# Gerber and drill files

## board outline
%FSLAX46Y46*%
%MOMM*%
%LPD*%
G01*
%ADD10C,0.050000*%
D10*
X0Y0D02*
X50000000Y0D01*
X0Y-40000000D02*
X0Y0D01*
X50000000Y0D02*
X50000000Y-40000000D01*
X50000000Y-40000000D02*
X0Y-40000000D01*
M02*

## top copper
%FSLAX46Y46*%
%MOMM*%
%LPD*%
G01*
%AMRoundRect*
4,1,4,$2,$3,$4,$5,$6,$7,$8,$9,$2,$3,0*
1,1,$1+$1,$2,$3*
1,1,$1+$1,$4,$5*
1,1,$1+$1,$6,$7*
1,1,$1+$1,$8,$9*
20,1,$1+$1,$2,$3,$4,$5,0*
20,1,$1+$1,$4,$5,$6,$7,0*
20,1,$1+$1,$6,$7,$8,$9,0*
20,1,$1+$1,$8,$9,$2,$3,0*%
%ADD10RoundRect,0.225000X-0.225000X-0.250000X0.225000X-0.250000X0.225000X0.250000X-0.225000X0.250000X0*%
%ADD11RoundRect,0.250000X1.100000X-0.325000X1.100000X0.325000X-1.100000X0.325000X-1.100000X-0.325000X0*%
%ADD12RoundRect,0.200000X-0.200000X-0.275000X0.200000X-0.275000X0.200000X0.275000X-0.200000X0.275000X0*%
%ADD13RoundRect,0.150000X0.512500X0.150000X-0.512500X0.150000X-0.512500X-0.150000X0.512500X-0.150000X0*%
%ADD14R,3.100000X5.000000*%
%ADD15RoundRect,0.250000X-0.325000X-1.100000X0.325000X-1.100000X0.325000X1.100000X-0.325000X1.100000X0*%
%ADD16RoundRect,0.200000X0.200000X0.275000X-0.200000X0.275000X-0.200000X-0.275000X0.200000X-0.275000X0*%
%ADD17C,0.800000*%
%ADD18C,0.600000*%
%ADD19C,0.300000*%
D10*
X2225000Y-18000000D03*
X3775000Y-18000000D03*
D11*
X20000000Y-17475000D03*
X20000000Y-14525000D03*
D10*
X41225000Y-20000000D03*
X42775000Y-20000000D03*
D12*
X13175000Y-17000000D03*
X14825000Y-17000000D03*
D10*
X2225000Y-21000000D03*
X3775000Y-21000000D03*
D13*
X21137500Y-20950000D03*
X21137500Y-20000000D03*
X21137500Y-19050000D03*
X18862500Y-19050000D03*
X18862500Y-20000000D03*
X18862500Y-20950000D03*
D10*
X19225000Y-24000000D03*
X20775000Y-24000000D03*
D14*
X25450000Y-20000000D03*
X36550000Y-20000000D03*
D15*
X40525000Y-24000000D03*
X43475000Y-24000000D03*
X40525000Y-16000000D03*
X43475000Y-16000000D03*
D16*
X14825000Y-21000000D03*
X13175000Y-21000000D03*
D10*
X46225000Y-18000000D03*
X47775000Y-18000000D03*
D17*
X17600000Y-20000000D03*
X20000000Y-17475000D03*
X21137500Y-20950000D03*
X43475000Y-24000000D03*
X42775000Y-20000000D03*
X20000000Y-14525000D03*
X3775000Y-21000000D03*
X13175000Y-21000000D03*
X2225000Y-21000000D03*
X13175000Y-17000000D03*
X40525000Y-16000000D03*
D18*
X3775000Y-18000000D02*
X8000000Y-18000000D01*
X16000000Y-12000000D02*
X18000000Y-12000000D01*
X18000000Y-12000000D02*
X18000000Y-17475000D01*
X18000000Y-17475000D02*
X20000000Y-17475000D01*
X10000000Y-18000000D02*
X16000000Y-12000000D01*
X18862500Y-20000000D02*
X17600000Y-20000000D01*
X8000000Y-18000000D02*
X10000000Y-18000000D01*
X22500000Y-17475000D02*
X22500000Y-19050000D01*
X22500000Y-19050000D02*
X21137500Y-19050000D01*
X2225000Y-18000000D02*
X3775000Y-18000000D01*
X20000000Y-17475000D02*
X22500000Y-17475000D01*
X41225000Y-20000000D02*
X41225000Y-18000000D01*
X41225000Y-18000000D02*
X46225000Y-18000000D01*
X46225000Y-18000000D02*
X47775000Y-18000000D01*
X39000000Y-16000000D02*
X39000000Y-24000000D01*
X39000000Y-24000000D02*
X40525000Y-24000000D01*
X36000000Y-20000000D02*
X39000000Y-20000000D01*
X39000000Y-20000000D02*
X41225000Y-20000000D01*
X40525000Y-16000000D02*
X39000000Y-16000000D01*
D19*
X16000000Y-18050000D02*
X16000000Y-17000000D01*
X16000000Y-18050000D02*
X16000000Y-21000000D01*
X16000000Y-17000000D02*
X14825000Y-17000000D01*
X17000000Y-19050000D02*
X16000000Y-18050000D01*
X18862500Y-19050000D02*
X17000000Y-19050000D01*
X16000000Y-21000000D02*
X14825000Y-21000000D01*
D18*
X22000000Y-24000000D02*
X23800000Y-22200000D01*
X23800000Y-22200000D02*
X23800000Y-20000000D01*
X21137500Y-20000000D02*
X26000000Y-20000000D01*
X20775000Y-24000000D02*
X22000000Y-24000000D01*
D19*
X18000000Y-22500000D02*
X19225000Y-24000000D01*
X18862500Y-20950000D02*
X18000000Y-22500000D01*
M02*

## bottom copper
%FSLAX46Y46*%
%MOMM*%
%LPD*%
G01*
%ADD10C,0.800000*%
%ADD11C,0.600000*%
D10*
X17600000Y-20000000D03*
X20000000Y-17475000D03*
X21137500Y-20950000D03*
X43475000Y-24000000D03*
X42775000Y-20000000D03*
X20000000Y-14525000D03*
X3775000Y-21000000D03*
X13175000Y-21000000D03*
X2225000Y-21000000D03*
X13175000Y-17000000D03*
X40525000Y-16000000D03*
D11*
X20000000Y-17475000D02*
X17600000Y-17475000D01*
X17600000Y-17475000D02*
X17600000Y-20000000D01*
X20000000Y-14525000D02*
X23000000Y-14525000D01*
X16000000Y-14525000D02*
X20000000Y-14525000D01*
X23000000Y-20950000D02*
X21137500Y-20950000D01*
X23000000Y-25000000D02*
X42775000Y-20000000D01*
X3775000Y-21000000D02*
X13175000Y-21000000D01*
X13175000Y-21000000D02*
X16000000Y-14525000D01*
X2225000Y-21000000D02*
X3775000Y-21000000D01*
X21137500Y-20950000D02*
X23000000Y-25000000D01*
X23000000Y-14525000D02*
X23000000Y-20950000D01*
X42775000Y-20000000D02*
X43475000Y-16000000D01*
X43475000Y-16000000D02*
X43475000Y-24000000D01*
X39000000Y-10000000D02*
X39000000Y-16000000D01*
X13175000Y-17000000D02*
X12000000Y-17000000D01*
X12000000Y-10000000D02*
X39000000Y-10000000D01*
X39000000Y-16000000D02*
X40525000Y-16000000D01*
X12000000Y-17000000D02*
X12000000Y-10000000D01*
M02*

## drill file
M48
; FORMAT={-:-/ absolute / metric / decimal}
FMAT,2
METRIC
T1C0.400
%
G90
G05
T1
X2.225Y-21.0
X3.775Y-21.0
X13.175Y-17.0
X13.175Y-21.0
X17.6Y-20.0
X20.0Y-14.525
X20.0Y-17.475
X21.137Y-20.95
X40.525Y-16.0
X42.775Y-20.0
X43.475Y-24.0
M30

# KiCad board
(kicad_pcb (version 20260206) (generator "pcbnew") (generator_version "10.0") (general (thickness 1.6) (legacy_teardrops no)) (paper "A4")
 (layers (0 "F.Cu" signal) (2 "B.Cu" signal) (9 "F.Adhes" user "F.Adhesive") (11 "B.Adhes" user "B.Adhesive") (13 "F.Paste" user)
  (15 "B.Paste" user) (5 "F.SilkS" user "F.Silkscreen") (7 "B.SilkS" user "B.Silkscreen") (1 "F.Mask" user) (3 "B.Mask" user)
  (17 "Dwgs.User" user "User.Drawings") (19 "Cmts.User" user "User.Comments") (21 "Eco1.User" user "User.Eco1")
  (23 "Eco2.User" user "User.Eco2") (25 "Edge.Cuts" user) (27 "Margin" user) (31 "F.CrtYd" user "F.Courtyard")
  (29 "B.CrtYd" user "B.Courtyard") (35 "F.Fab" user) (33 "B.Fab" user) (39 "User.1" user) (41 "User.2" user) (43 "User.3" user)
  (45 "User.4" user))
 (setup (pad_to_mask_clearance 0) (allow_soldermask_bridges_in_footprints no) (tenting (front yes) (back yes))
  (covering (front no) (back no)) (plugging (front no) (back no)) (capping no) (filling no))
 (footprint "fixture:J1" (layer "F.Cu") (at 3 18)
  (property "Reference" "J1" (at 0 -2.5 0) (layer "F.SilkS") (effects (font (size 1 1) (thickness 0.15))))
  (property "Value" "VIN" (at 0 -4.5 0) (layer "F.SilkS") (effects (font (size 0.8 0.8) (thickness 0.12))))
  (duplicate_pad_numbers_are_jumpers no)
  (pad "1" smd roundrect (at -0.775 0) (size 0.9 0.95) (layers "F.Cu" "F.Mask" "F.Paste") (roundrect_rratio 0.25) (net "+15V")
   (thermal_bridge_angle 45))
  (pad "2" smd roundrect (at 0.775 0) (size 0.9 0.95) (layers "F.Cu" "F.Mask" "F.Paste") (roundrect_rratio 0.25) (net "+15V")
   (thermal_bridge_angle 45)))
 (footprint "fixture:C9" (layer "F.Cu") (at 20 16 90)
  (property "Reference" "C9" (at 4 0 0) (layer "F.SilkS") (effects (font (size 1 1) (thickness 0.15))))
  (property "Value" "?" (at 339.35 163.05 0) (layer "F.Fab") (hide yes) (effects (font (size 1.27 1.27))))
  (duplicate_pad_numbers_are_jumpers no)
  (pad "1" smd roundrect (at -1.475 0 90) (size 1.15 2.7) (layers "F.Cu" "F.Mask" "F.Paste") (roundrect_rratio 0.217391) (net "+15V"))
  (pad "2" smd roundrect (at 1.475 0 90) (size 1.15 2.7) (layers "F.Cu" "F.Mask" "F.Paste") (roundrect_rratio 0.217391) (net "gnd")))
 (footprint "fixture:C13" (layer "F.Cu") (at 42 20)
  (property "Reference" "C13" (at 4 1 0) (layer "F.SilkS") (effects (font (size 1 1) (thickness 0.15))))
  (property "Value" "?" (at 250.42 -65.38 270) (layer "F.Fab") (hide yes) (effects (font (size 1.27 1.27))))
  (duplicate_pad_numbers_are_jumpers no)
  (pad "1" smd roundrect (at -0.775 0) (size 0.9 0.95) (layers "F.Cu" "F.Mask" "F.Paste") (roundrect_rratio 0.25) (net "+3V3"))
  (pad "2" smd roundrect (at 0.775 0) (size 0.9 0.95) (layers "F.Cu" "F.Mask" "F.Paste") (roundrect_rratio 0.25) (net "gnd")))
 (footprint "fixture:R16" (layer "F.Cu") (at 14 17)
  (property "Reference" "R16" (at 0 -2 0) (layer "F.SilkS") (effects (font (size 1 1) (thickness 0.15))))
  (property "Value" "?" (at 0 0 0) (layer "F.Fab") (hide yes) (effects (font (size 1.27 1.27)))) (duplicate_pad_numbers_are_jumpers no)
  (pad "1" smd roundrect (at -0.825 0) (size 0.8 0.95) (layers "F.Cu" "F.Mask" "F.Paste") (roundrect_rratio 0.25) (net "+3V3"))
  (pad "2" smd roundrect (at 0.825 0) (size 0.8 0.95) (layers "F.Cu" "F.Mask" "F.Paste") (roundrect_rratio 0.25) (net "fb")))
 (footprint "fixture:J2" (layer "F.Cu") (at 3 21)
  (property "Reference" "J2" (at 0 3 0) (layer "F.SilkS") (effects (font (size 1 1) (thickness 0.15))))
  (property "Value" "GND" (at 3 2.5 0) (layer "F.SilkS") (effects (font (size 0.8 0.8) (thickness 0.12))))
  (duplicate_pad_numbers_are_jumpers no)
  (pad "1" smd roundrect (at -0.775 0) (size 0.9 0.95) (layers "F.Cu" "F.Mask" "F.Paste") (roundrect_rratio 0.25) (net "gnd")
   (thermal_bridge_angle 45))
  (pad "2" smd roundrect (at 0.775 0) (size 0.9 0.95) (layers "F.Cu" "F.Mask" "F.Paste") (roundrect_rratio 0.25) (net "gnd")
   (thermal_bridge_angle 45)))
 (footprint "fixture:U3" (layer "F.Cu") (at 20 20 180)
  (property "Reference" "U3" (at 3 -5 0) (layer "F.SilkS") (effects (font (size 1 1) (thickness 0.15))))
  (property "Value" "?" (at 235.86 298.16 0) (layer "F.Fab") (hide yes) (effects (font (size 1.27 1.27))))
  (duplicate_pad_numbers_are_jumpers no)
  (pad "1" smd roundrect (at -1.1375 -0.95 180) (size 1.325 0.6) (layers "F.Cu" "F.Mask" "F.Paste") (roundrect_rratio 0.25) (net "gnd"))
  (pad "2" smd roundrect (at -1.1375 0 180) (size 1.325 0.6) (layers "F.Cu" "F.Mask" "F.Paste") (roundrect_rratio 0.25) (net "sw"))
  (pad "3" smd roundrect (at -1.1375 0.95 180) (size 1.325 0.6) (layers "F.Cu" "F.Mask" "F.Paste") (roundrect_rratio 0.25) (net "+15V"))
  (pad "4" smd roundrect (at 1.1375 0.95 180) (size 1.325 0.6) (layers "F.Cu" "F.Mask" "F.Paste") (roundrect_rratio 0.25) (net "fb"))
  (pad "5" smd roundrect (at 1.1375 0 180) (size 1.325 0.6) (layers "F.Cu" "F.Mask" "F.Paste") (roundrect_rratio 0.25) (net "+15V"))
  (pad "6" smd roundrect (at 1.1375 -0.95 180) (size 1.325 0.6) (layers "F.Cu" "F.Mask" "F.Paste") (roundrect_rratio 0.25) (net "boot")))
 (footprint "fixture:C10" (layer "F.Cu") (at 20 24)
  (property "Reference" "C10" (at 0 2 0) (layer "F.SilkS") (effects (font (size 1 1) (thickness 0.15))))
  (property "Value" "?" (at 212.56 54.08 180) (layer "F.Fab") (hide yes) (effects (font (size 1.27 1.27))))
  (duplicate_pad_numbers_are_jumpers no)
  (pad "1" smd roundrect (at -0.775 0) (size 0.9 0.95) (layers "F.Cu" "F.Mask" "F.Paste") (roundrect_rratio 0.25) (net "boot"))
  (pad "2" smd roundrect (at 0.775 0) (size 0.9 0.95) (layers "F.Cu" "F.Mask" "F.Paste") (roundrect_rratio 0.25) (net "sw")))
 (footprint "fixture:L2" (layer "F.Cu") (at 31 20)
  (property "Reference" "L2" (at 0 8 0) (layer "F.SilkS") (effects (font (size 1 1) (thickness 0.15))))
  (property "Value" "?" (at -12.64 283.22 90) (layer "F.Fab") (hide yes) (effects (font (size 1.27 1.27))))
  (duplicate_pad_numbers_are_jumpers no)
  (pad "1" smd rect (at -5.55 0) (size 3.1 5) (layers "F.Cu" "F.Mask" "F.Paste") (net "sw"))
  (pad "2" smd rect (at 5.55 0) (size 3.1 5) (layers "F.Cu" "F.Mask" "F.Paste") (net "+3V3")))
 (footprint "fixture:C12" (layer "F.Cu") (at 42 24)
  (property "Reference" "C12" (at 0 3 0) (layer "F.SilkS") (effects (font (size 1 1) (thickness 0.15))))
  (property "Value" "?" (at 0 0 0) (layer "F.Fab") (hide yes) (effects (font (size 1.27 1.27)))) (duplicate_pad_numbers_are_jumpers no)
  (pad "1" smd roundrect (at -1.475 0) (size 1.15 2.7) (layers "F.Cu" "F.Mask" "F.Paste") (roundrect_rratio 0.217391) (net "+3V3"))
  (pad "2" smd roundrect (at 1.475 0) (size 1.15 2.7) (layers "F.Cu" "F.Mask" "F.Paste") (roundrect_rratio 0.217391) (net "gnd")))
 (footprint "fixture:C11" (layer "F.Cu") (at 42 16)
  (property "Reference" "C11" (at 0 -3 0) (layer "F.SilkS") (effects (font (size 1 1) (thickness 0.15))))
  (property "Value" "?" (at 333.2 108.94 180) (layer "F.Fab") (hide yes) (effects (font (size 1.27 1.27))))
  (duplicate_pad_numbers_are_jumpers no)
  (pad "1" smd roundrect (at -1.475 0) (size 1.15 2.7) (layers "F.Cu" "F.Mask" "F.Paste") (roundrect_rratio 0.217391) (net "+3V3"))
  (pad "2" smd roundrect (at 1.475 0) (size 1.15 2.7) (layers "F.Cu" "F.Mask" "F.Paste") (roundrect_rratio 0.217391) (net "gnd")))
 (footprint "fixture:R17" (layer "F.Cu") (at 14 21 180)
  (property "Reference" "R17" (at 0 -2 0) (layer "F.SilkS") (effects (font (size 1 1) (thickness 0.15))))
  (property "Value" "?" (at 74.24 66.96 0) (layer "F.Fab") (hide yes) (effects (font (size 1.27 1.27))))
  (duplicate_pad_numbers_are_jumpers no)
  (pad "1" smd roundrect (at -0.825 0 180) (size 0.8 0.95) (layers "F.Cu" "F.Mask" "F.Paste") (roundrect_rratio 0.25) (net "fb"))
  (pad "2" smd roundrect (at 0.825 0 180) (size 0.8 0.95) (layers "F.Cu" "F.Mask" "F.Paste") (roundrect_rratio 0.25) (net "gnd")))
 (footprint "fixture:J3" (layer "F.Cu") (at 47 18)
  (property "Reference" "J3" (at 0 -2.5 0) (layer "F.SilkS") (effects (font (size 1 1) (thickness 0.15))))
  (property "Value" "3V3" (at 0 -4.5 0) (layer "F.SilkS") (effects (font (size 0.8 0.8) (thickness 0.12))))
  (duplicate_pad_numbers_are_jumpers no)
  (pad "1" smd roundrect (at -0.775 0) (size 0.9 0.95) (layers "F.Cu" "F.Mask" "F.Paste") (roundrect_rratio 0.25) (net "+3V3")
   (thermal_bridge_angle 45))
  (pad "2" smd roundrect (at 0.775 0) (size 0.9 0.95) (layers "F.Cu" "F.Mask" "F.Paste") (roundrect_rratio 0.25) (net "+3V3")
   (thermal_bridge_angle 45)))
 (gr_line (start 0 0) (end 50 0) (stroke (width 0.05) (type default)) (layer "Edge.Cuts"))
 (gr_line (start 0 40) (end 0 0) (stroke (width 0.05) (type default)) (layer "Edge.Cuts"))
 (gr_line (start 50 0) (end 50 40) (stroke (width 0.05) (type default)) (layer "Edge.Cuts"))
 (gr_line (start 50 40) (end 0 40) (stroke (width 0.05) (type default)) (layer "Edge.Cuts"))
 (segment (start 3.775 18) (end 8 18) (width 0.6) (layer "F.Cu") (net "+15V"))
 (segment (start 16 12) (end 18 12) (width 0.6) (layer "F.Cu") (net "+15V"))
 (segment (start 18 12) (end 18 17.475) (width 0.6) (layer "F.Cu") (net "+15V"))
 (segment (start 18 17.475) (end 20 17.475) (width 0.6) (layer "F.Cu") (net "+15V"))
 (segment (start 10 18) (end 16 12) (width 0.6) (layer "F.Cu") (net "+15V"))
 (segment (start 18.8625 20) (end 17.6 20) (width 0.6) (layer "F.Cu") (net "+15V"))
 (segment (start 8 18) (end 10 18) (width 0.6) (layer "F.Cu") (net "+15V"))
 (segment (start 22.5 17.475) (end 22.5 19.05) (width 0.6) (layer "F.Cu") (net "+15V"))
 (segment (start 22.5 19.05) (end 21.1375 19.05) (width 0.6) (layer "F.Cu") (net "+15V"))
 (segment (start 2.225 18) (end 3.775 18) (width 0.6) (layer "F.Cu") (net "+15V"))
 (segment (start 20 17.475) (end 22.5 17.475) (width 0.6) (layer "F.Cu") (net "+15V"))
 (via (at 17.6 20) (size 0.8) (drill 0.4) (layers "F.Cu" "B.Cu") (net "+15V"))
 (via (at 20 17.475) (size 0.8) (drill 0.4) (layers "F.Cu" "B.Cu") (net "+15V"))
 (segment (start 20 17.475) (end 17.6 17.475) (width 0.6) (layer "B.Cu") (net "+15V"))
 (segment (start 17.6 17.475) (end 17.6 20) (width 0.6) (layer "B.Cu") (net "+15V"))
 (via (at 21.1375 20.95) (size 0.8) (drill 0.4) (layers "F.Cu" "B.Cu") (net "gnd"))
 (via (at 43.475 24) (size 0.8) (drill 0.4) (layers "F.Cu" "B.Cu") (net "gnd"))
 (via (at 42.775 20) (size 0.8) (drill 0.4) (layers "F.Cu" "B.Cu") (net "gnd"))
 (via (at 20 14.525) (size 0.8) (drill 0.4) (layers "F.Cu" "B.Cu") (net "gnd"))
 (via (at 3.775 21) (size 0.8) (drill 0.4) (layers "F.Cu" "B.Cu") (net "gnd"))
 (via (at 13.175 21) (size 0.8) (drill 0.4) (layers "F.Cu" "B.Cu") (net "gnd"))
 (via (at 2.225 21) (size 0.8) (drill 0.4) (layers "F.Cu" "B.Cu") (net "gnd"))
 (segment (start 20 14.525) (end 23 14.525) (width 0.6) (layer "B.Cu") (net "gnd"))
 (segment (start 16 14.525) (end 20 14.525) (width 0.6) (layer "B.Cu") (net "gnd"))
 (segment (start 23 20.95) (end 21.1375 20.95) (width 0.6) (layer "B.Cu") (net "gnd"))
 (segment (start 23 25) (end 42.775 20) (width 0.6) (layer "B.Cu") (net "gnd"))
 (segment (start 3.775 21) (end 13.175 21) (width 0.6) (layer "B.Cu") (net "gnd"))
 (segment (start 13.175 21) (end 16 14.525) (width 0.6) (layer "B.Cu") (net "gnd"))
 (segment (start 2.225 21) (end 3.775 21) (width 0.6) (layer "B.Cu") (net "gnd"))
 (segment (start 21.1375 20.95) (end 23 25) (width 0.6) (layer "B.Cu") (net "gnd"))
 (segment (start 23 14.525) (end 23 20.95) (width 0.6) (layer "B.Cu") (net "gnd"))
 (segment (start 42.775 20) (end 43.475 16) (width 0.6) (layer "B.Cu") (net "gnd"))
 (segment (start 43.475 16) (end 43.475 24) (width 0.6) (layer "B.Cu") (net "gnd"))
 (segment (start 41.225 20) (end 41.225 18) (width 0.6) (layer "F.Cu") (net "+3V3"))
 (segment (start 41.225 18) (end 46.225 18) (width 0.6) (layer "F.Cu") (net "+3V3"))
 (segment (start 46.225 18) (end 47.775 18) (width 0.6) (layer "F.Cu") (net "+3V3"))
 (segment (start 39 16) (end 39 24) (width 0.6) (layer "F.Cu") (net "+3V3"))
 (segment (start 39 24) (end 40.525 24) (width 0.6) (layer "F.Cu") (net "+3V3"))
 (segment (start 36 20) (end 39 20) (width 0.6) (layer "F.Cu") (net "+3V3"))
 (segment (start 39 20) (end 41.225 20) (width 0.6) (layer "F.Cu") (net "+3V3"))
 (segment (start 40.525 16) (end 39 16) (width 0.6) (layer "F.Cu") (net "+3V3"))
 (via (at 13.175 17) (size 0.8) (drill 0.4) (layers "F.Cu" "B.Cu") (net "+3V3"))
 (via (at 40.525 16) (size 0.8) (drill 0.4) (layers "F.Cu" "B.Cu") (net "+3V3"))
 (segment (start 39 10) (end 39 16) (width 0.6) (layer "B.Cu") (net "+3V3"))
 (segment (start 13.175 17) (end 12 17) (width 0.6) (layer "B.Cu") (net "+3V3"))
 (segment (start 12 10) (end 39 10) (width 0.6) (layer "B.Cu") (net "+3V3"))
 (segment (start 39 16) (end 40.525 16) (width 0.6) (layer "B.Cu") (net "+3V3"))
 (segment (start 12 17) (end 12 10) (width 0.6) (layer "B.Cu") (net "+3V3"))
 (segment (start 16 18.05) (end 16 17) (width 0.3) (layer "F.Cu") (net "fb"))
 (segment (start 16 18.05) (end 16 21) (width 0.3) (layer "F.Cu") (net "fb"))
 (segment (start 16 17) (end 14.825 17) (width 0.3) (layer "F.Cu") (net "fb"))
 (segment (start 17 19.05) (end 16 18.05) (width 0.3) (layer "F.Cu") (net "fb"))
 (segment (start 18.8625 19.05) (end 17 19.05) (width 0.3) (layer "F.Cu") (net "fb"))
 (segment (start 16 21) (end 14.825 21) (width 0.3) (layer "F.Cu") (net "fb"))
 (segment (start 22 24) (end 23.8 22.2) (width 0.6) (layer "F.Cu") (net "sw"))
 (segment (start 23.8 22.2) (end 23.8 20) (width 0.6) (layer "F.Cu") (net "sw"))
 (segment (start 21.1375 20) (end 26 20) (width 0.6) (layer "F.Cu") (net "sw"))
 (segment (start 20.775 24) (end 22 24) (width 0.6) (layer "F.Cu") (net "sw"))
 (segment (start 18 22.5) (end 19.225 24) (width 0.3) (layer "F.Cu") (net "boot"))
 (segment (start 18.8625 20.95) (end 18 22.5) (width 0.3) (layer "F.Cu") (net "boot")))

